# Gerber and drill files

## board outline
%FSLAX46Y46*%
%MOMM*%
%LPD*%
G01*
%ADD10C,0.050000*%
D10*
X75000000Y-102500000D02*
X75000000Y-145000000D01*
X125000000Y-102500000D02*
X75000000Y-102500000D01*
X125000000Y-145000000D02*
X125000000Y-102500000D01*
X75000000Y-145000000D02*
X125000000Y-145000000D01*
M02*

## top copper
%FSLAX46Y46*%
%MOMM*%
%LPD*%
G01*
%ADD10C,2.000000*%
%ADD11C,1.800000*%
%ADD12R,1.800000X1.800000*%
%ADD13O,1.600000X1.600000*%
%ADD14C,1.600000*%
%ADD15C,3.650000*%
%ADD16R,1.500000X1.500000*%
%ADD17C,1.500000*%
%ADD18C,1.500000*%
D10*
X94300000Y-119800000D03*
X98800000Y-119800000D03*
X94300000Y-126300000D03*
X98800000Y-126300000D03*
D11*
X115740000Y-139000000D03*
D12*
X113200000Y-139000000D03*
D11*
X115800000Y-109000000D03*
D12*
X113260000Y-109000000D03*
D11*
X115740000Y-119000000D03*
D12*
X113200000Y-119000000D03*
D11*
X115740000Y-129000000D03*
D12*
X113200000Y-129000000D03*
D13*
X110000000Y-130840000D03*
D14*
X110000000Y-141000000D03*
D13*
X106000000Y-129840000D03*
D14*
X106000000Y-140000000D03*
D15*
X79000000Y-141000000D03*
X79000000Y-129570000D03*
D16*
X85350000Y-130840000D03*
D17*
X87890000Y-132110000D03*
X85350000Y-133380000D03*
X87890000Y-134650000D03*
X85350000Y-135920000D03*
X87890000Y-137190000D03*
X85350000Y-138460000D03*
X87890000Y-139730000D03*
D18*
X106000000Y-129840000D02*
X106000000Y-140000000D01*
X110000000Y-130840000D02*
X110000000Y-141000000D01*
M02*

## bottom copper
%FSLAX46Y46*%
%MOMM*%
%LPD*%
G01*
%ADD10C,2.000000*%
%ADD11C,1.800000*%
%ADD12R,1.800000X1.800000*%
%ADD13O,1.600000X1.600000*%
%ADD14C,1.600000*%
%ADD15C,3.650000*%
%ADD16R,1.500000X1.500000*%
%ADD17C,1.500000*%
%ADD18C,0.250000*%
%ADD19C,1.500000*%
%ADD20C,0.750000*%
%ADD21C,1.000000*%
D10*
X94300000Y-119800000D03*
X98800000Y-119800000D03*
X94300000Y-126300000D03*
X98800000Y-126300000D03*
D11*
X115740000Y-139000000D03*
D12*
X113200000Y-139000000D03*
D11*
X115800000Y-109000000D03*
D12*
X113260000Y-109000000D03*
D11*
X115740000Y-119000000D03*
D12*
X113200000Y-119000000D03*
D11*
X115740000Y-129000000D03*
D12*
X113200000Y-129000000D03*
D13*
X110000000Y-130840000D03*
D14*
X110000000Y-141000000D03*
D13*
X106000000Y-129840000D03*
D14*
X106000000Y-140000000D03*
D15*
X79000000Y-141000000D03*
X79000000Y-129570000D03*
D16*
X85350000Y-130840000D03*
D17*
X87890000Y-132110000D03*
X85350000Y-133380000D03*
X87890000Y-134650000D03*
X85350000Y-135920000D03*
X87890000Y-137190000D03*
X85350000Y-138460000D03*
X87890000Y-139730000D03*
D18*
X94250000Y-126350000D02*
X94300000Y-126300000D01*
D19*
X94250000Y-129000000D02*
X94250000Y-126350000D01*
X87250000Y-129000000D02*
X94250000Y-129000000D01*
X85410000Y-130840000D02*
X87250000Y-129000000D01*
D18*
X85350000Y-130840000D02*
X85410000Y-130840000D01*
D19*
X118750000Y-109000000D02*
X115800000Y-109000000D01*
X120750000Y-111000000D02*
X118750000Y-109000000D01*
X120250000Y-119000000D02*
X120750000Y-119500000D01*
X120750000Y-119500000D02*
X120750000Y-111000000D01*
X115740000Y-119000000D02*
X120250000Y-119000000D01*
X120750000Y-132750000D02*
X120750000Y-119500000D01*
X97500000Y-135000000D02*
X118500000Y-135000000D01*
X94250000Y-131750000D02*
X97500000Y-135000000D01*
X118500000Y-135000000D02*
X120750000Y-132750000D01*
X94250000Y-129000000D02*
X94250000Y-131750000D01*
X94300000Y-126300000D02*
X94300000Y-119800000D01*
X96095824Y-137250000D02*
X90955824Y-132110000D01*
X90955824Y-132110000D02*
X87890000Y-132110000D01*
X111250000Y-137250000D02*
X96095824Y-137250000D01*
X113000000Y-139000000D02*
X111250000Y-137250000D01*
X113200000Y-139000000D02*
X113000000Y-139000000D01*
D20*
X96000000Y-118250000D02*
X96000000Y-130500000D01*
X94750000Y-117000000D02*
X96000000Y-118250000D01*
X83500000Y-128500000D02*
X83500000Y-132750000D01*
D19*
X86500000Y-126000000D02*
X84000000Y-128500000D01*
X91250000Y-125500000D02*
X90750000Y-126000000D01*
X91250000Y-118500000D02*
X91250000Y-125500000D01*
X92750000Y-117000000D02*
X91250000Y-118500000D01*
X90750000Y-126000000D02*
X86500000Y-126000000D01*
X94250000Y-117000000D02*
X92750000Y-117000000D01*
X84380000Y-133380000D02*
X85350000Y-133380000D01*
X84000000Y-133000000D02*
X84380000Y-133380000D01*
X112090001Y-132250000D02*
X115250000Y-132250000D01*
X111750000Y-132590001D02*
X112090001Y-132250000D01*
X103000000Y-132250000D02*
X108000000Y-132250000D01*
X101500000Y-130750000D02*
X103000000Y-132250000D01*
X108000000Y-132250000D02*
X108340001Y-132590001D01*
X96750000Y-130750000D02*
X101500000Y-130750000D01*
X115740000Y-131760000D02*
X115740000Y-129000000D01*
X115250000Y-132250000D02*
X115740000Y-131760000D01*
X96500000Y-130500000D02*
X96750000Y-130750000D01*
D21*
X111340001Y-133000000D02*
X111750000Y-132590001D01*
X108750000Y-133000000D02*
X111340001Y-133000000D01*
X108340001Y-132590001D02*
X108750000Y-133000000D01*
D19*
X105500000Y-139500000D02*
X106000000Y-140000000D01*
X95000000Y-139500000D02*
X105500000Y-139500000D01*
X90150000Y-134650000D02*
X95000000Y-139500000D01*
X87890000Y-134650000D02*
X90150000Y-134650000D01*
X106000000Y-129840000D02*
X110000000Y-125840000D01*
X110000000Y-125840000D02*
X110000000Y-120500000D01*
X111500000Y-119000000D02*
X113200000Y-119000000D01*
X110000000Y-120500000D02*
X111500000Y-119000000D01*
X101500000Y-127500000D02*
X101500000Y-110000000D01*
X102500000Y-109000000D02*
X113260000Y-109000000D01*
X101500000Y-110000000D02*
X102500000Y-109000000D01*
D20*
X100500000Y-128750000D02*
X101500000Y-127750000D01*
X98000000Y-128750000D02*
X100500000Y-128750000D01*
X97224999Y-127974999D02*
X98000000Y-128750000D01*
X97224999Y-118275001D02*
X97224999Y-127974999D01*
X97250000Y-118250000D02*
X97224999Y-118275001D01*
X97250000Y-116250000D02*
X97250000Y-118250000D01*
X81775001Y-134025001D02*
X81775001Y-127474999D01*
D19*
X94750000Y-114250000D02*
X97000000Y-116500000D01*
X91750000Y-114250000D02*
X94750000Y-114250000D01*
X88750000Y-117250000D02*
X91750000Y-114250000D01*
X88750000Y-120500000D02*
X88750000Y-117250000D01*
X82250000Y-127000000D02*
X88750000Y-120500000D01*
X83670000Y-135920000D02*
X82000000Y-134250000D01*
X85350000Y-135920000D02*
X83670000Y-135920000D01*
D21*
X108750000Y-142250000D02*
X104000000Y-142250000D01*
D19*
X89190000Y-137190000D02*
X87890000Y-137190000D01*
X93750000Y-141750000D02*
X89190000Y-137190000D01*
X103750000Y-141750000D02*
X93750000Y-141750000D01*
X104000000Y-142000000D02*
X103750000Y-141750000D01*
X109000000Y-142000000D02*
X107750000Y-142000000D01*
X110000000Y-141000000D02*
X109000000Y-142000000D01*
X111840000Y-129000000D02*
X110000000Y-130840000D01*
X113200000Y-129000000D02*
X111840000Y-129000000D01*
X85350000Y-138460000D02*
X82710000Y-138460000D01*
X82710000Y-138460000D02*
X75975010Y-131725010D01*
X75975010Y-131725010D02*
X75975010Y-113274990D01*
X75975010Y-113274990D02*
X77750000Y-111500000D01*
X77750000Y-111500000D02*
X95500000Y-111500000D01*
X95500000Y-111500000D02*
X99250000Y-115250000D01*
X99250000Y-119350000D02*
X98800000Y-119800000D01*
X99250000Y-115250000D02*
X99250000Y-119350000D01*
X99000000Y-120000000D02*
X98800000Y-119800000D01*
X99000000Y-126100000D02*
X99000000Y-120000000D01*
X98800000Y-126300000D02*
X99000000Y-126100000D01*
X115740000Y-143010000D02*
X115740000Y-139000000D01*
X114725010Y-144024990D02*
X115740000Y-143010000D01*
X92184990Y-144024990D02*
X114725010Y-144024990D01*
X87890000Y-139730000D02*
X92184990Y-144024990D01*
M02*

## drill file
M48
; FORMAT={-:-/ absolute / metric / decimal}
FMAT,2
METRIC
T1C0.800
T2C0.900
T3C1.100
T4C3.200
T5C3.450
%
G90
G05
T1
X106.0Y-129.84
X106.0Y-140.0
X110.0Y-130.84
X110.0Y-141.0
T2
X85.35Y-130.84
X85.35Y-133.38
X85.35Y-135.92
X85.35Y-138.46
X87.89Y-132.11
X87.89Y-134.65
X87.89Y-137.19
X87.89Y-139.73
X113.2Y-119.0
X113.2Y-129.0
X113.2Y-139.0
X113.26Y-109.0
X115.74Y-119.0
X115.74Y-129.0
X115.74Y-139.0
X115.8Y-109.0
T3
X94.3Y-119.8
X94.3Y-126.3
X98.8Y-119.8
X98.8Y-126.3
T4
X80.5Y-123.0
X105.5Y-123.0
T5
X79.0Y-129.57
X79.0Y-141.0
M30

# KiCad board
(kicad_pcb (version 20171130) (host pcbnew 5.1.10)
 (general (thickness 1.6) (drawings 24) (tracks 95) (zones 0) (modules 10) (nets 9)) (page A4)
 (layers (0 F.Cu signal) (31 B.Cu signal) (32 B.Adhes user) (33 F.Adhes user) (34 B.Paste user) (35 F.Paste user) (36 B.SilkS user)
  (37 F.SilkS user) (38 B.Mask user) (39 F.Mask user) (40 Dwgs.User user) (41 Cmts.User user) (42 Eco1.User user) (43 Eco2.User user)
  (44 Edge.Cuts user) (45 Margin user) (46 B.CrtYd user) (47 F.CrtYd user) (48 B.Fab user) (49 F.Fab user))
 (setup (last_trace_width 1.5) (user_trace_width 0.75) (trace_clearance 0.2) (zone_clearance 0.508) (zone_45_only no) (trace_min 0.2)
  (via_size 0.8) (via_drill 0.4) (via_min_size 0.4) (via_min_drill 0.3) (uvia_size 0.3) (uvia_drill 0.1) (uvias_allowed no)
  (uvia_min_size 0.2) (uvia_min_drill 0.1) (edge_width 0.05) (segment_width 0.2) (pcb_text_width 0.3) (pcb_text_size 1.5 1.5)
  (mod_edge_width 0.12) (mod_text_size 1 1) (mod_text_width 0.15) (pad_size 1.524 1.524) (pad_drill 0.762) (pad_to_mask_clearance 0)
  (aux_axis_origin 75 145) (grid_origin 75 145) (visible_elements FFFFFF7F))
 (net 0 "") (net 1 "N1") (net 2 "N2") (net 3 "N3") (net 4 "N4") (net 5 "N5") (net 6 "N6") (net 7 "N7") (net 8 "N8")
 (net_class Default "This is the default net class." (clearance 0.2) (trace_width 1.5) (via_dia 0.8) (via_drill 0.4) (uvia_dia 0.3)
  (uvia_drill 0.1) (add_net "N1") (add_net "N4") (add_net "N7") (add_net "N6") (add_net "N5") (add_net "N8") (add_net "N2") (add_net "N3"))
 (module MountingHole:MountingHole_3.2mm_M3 (layer F.Cu) (at 105.5 123)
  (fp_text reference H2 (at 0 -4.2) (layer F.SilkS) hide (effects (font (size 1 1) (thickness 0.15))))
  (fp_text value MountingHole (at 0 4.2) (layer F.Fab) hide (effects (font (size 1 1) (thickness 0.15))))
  (pad 1 np_thru_hole circle (at 0 0) (size 3.2 3.2) (drill 3.2) (layers *.Cu *.Mask)))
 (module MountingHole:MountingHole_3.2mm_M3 (layer F.Cu) (at 80.5 123)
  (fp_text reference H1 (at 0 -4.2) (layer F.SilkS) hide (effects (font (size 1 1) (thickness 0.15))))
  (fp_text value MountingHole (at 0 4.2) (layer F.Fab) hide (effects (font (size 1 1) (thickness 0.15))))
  (pad 1 np_thru_hole circle (at 0 0) (size 3.2 3.2) (drill 3.2) (layers *.Cu *.Mask)))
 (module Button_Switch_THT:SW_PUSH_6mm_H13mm (layer F.Cu) (at 94.3 126.3 90)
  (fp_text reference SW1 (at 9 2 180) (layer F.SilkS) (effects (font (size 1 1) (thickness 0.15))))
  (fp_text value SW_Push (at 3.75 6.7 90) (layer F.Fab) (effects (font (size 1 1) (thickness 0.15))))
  (pad 1 thru_hole circle (at 6.5 0 180) (size 2 2) (drill 1.1) (layers *.Cu *.Mask) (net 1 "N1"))
  (pad 2 thru_hole circle (at 6.5 4.5 180) (size 2 2) (drill 1.1) (layers *.Cu *.Mask) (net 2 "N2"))
  (pad 1 thru_hole circle (at 0 0 180) (size 2 2) (drill 1.1) (layers *.Cu *.Mask) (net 1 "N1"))
  (pad 2 thru_hole circle (at 0 4.5 180) (size 2 2) (drill 1.1) (layers *.Cu *.Mask) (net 2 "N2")))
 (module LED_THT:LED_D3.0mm (layer F.Cu) (at 113.2 139)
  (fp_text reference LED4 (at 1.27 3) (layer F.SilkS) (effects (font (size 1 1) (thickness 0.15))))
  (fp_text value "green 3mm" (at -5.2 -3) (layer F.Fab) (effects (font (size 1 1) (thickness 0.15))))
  (pad 2 thru_hole circle (at 2.54 0) (size 1.8 1.8) (drill 0.9) (layers *.Cu *.Mask) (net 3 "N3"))
  (pad 1 thru_hole rect (at 0 0) (size 1.8 1.8) (drill 0.9) (layers *.Cu *.Mask) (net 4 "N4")))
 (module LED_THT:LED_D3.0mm (layer F.Cu) (at 113.26 109)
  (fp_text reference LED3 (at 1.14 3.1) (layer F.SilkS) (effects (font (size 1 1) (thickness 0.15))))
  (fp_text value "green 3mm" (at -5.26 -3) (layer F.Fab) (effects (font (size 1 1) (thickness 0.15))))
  (pad 2 thru_hole circle (at 2.54 0) (size 1.8 1.8) (drill 0.9) (layers *.Cu *.Mask) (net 1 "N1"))
  (pad 1 thru_hole rect (at 0 0) (size 1.8 1.8) (drill 0.9) (layers *.Cu *.Mask) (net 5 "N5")))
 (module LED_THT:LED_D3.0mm (layer F.Cu) (at 113.2 119)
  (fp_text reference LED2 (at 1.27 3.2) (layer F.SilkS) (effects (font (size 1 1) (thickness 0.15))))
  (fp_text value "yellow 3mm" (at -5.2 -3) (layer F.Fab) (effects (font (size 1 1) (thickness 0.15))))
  (pad 2 thru_hole circle (at 2.54 0) (size 1.8 1.8) (drill 0.9) (layers *.Cu *.Mask) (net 1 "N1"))
  (pad 1 thru_hole rect (at 0 0) (size 1.8 1.8) (drill 0.9) (layers *.Cu *.Mask) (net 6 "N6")))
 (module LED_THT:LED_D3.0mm (layer F.Cu) (at 113.2 129)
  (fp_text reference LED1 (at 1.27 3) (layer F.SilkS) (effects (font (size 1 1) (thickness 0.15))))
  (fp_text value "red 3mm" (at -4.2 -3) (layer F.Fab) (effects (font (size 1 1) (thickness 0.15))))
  (pad 2 thru_hole circle (at 2.54 0) (size 1.8 1.8) (drill 0.9) (layers *.Cu *.Mask) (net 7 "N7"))
  (pad 1 thru_hole rect (at 0 0) (size 1.8 1.8) (drill 0.9) (layers *.Cu *.Mask) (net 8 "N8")))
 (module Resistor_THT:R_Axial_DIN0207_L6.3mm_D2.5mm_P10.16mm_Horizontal (layer F.Cu) (at 110 141 90)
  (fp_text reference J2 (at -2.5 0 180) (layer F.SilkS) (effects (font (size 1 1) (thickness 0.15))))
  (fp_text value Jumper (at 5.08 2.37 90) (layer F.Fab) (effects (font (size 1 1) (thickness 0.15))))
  (pad 2 thru_hole oval (at 10.16 0 90) (size 1.6 1.6) (drill 0.8) (layers *.Cu *.Mask) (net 8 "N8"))
  (pad 1 thru_hole circle (at 0 0 90) (size 1.6 1.6) (drill 0.8) (layers *.Cu *.Mask) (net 8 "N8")))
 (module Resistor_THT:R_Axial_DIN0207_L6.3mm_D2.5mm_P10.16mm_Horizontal (layer F.Cu) (at 106 140 90)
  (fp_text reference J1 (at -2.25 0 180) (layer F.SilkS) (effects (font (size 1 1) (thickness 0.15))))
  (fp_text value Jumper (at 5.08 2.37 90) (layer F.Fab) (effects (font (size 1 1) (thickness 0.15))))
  (pad 2 thru_hole oval (at 10.16 0 90) (size 1.6 1.6) (drill 0.8) (layers *.Cu *.Mask) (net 6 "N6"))
  (pad 1 thru_hole circle (at 0 0 90) (size 1.6 1.6) (drill 0.8) (layers *.Cu *.Mask) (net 6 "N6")))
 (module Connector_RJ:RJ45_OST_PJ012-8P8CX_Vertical (layer F.Cu) (at 85.35 130.84 270)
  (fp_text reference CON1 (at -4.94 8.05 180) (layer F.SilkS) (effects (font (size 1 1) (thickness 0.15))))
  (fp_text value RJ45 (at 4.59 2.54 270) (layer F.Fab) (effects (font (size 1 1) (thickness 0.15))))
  (pad "" np_thru_hole circle (at 10.16 6.35 270) (size 3.65 3.65) (drill 3.45) (layers *.Cu *.SilkS *.Mask))
  (pad "" np_thru_hole circle (at -1.27 6.35 270) (size 3.65 3.65) (drill 3.45) (layers *.Cu *.SilkS *.Mask))
  (pad 1 thru_hole rect (at 0 0 270) (size 1.5 1.5) (drill 0.9) (layers *.Cu *.Mask) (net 1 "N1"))
  (pad 2 thru_hole circle (at 1.27 -2.54 270) (size 1.5 1.5) (drill 0.9) (layers *.Cu *.Mask) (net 4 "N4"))
  (pad 3 thru_hole circle (at 2.54 0 270) (size 1.5 1.5) (drill 0.9) (layers *.Cu *.Mask) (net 7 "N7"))
  (pad 4 thru_hole circle (at 3.81 -2.54 270) (size 1.5 1.5) (drill 0.9) (layers *.Cu *.Mask) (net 6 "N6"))
  (pad 5 thru_hole circle (at 5.08 0 270) (size 1.5 1.5) (drill 0.9) (layers *.Cu *.Mask) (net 5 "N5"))
  (pad 6 thru_hole circle (at 6.35 -2.54 270) (size 1.5 1.5) (drill 0.9) (layers *.Cu *.Mask) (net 8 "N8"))
  (pad 7 thru_hole circle (at 7.62 0 270) (size 1.5 1.5) (drill 0.9) (layers *.Cu *.Mask) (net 2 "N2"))
  (pad 8 thru_hole circle (at 8.89 -2.54 270) (size 1.5 1.5) (drill 0.9) (layers *.Cu *.Mask) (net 3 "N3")))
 (gr_line (start 75 102.5) (end 75 145) (layer Edge.Cuts) (width 0.05))
 (gr_line (start 125 102.5) (end 75 102.5) (layer Edge.Cuts) (width 0.05))
 (gr_line (start 125 145) (end 125 102.5) (layer Edge.Cuts) (width 0.05))
 (gr_line (start 75 145) (end 125 145) (layer Edge.Cuts) (width 0.05))
 (segment (start 94.25 126.35) (end 94.3 126.3) (width 0.25) (layer B.Cu) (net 1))
 (segment (start 94.25 129) (end 94.25 126.35) (width 1.5) (layer B.Cu) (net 1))
 (segment (start 87.25 129) (end 94.25 129) (width 1.5) (layer B.Cu) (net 1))
 (segment (start 85.41 130.84) (end 87.25 129) (width 1.5) (layer B.Cu) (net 1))
 (segment (start 85.35 130.84) (end 85.41 130.84) (width 0.25) (layer B.Cu) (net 1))
 (segment (start 118.75 109) (end 115.8 109) (width 1.5) (layer B.Cu) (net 1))
 (segment (start 120.75 111) (end 118.75 109) (width 1.5) (layer B.Cu) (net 1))
 (segment (start 120.25 119) (end 120.75 119.5) (width 1.5) (layer B.Cu) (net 1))
 (segment (start 120.75 119.5) (end 120.75 111) (width 1.5) (layer B.Cu) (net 1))
 (segment (start 115.74 119) (end 120.25 119) (width 1.5) (layer B.Cu) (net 1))
 (segment (start 120.75 132.75) (end 120.75 119.5) (width 1.5) (layer B.Cu) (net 1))
 (segment (start 97.5 135) (end 118.5 135) (width 1.5) (layer B.Cu) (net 1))
 (segment (start 94.25 131.75) (end 97.5 135) (width 1.5) (layer B.Cu) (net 1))
 (segment (start 118.5 135) (end 120.75 132.75) (width 1.5) (layer B.Cu) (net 1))
 (segment (start 94.25 129) (end 94.25 131.75) (width 1.5) (layer B.Cu) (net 1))
 (segment (start 94.3 126.3) (end 94.3 119.8) (width 1.5) (layer B.Cu) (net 1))
 (segment (start 96.095824 137.25) (end 90.955824 132.11) (width 1.5) (layer B.Cu) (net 4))
 (segment (start 90.955824 132.11) (end 87.89 132.11) (width 1.5) (layer B.Cu) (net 4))
 (segment (start 111.25 137.25) (end 96.095824 137.25) (width 1.5) (layer B.Cu) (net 4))
 (segment (start 113 139) (end 111.25 137.25) (width 1.5) (layer B.Cu) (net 4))
 (segment (start 113.2 139) (end 113 139) (width 1.5) (layer B.Cu) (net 4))
 (segment (start 96 118.25) (end 96 130.5) (width 0.75) (layer B.Cu) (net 7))
 (segment (start 94.75 117) (end 96 118.25) (width 0.75) (layer B.Cu) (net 7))
 (segment (start 83.5 128.5) (end 83.5 132.75) (width 0.75) (layer B.Cu) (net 7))
 (segment (start 86.5 126) (end 84 128.5) (width 1.5) (layer B.Cu) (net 7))
 (segment (start 91.25 125.5) (end 90.75 126) (width 1.5) (layer B.Cu) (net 7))
 (segment (start 91.25 118.5) (end 91.25 125.5) (width 1.5) (layer B.Cu) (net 7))
 (segment (start 92.75 117) (end 91.25 118.5) (width 1.5) (layer B.Cu) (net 7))
 (segment (start 90.75 126) (end 86.5 126) (width 1.5) (layer B.Cu) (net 7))
 (segment (start 94.25 117) (end 92.75 117) (width 1.5) (layer B.Cu) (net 7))
 (segment (start 84.38 133.38) (end 85.35 133.38) (width 1.5) (layer B.Cu) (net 7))
 (segment (start 84 133) (end 84.38 133.38) (width 1.5) (layer B.Cu) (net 7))
 (segment (start 112.090001 132.25) (end 115.25 132.25) (width 1.5) (layer B.Cu) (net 7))
 (segment (start 111.75 132.590001) (end 112.090001 132.25) (width 1.5) (layer B.Cu) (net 7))
 (segment (start 103 132.25) (end 108 132.25) (width 1.5) (layer B.Cu) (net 7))
 (segment (start 101.5 130.75) (end 103 132.25) (width 1.5) (layer B.Cu) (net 7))
 (segment (start 108 132.25) (end 108.340001 132.590001) (width 1.5) (layer B.Cu) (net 7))
 (segment (start 96.75 130.75) (end 101.5 130.75) (width 1.5) (layer B.Cu) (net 7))
 (segment (start 115.74 131.76) (end 115.74 129) (width 1.5) (layer B.Cu) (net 7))
 (segment (start 115.25 132.25) (end 115.74 131.76) (width 1.5) (layer B.Cu) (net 7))
 (segment (start 96.5 130.5) (end 96.75 130.75) (width 1.5) (layer B.Cu) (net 7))
 (segment (start 111.340001 133) (end 111.75 132.590001) (width 1) (layer B.Cu) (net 7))
 (segment (start 108.75 133) (end 111.340001 133) (width 1) (layer B.Cu) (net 7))
 (segment (start 108.340001 132.590001) (end 108.75 133) (width 1) (layer B.Cu) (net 7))
 (segment (start 105.5 139.5) (end 106 140) (width 1.5) (layer B.Cu) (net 6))
 (segment (start 95 139.5) (end 105.5 139.5) (width 1.5) (layer B.Cu) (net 6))
 (segment (start 90.15 134.65) (end 95 139.5) (width 1.5) (layer B.Cu) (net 6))
 (segment (start 87.89 134.65) (end 90.15 134.65) (width 1.5) (layer B.Cu) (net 6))
 (segment (start 106 129.84) (end 110 125.84) (width 1.5) (layer B.Cu) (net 6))
 (segment (start 110 125.84) (end 110 120.5) (width 1.5) (layer B.Cu) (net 6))
 (segment (start 111.5 119) (end 113.2 119) (width 1.5) (layer B.Cu) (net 6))
 (segment (start 110 120.5) (end 111.5 119) (width 1.5) (layer B.Cu) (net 6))
 (segment (start 106 129.84) (end 106 140) (width 1.5) (layer F.Cu) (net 6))
 (segment (start 101.5 127.5) (end 101.5 110) (width 1.5) (layer B.Cu) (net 5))
 (segment (start 102.5 109) (end 113.26 109) (width 1.5) (layer B.Cu) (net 5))
 (segment (start 101.5 110) (end 102.5 109) (width 1.5) (layer B.Cu) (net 5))
 (segment (start 100.5 128.75) (end 101.5 127.75) (width 0.75) (layer B.Cu) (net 5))
 (segment (start 98 128.75) (end 100.5 128.75) (width 0.75) (layer B.Cu) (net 5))
 (segment (start 97.224999 127.974999) (end 98 128.75) (width 0.75) (layer B.Cu) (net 5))
 (segment (start 97.224999 118.275001) (end 97.224999 127.974999) (width 0.75) (layer B.Cu) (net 5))
 (segment (start 97.25 118.25) (end 97.224999 118.275001) (width 0.75) (layer B.Cu) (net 5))
 (segment (start 97.25 116.25) (end 97.25 118.25) (width 0.75) (layer B.Cu) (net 5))
 (segment (start 81.775001 134.025001) (end 81.775001 127.474999) (width 0.75) (layer B.Cu) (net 5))
 (segment (start 94.75 114.25) (end 97 116.5) (width 1.5) (layer B.Cu) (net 5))
 (segment (start 91.75 114.25) (end 94.75 114.25) (width 1.5) (layer B.Cu) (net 5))
 (segment (start 88.75 117.25) (end 91.75 114.25) (width 1.5) (layer B.Cu) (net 5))
 (segment (start 88.75 120.5) (end 88.75 117.25) (width 1.5) (layer B.Cu) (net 5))
 (segment (start 82.25 127) (end 88.75 120.5) (width 1.5) (layer B.Cu) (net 5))
 (segment (start 83.67 135.92) (end 82 134.25) (width 1.5) (layer B.Cu) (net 5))
 (segment (start 85.35 135.92) (end 83.67 135.92) (width 1.5) (layer B.Cu) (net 5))
 (segment (start 108.75 142.25) (end 104 142.25) (width 1) (layer B.Cu) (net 8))
 (segment (start 89.19 137.19) (end 87.89 137.19) (width 1.5) (layer B.Cu) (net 8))
 (segment (start 93.75 141.75) (end 89.19 137.19) (width 1.5) (layer B.Cu) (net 8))
 (segment (start 103.75 141.75) (end 93.75 141.75) (width 1.5) (layer B.Cu) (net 8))
 (segment (start 104 142) (end 103.75 141.75) (width 1.5) (layer B.Cu) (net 8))
 (segment (start 109 142) (end 107.75 142) (width 1.5) (layer B.Cu) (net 8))
 (segment (start 110 141) (end 109 142) (width 1.5) (layer B.Cu) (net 8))
 (segment (start 111.84 129) (end 110 130.84) (width 1.5) (layer B.Cu) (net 8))
 (segment (start 113.2 129) (end 111.84 129) (width 1.5) (layer B.Cu) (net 8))
 (segment (start 110 130.84) (end 110 141) (width 1.5) (layer F.Cu) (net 8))
 (segment (start 85.35 138.46) (end 82.71 138.46) (width 1.5) (layer B.Cu) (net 2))
 (segment (start 82.71 138.46) (end 75.97501 131.72501) (width 1.5) (layer B.Cu) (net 2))
 (segment (start 75.97501 131.72501) (end 75.97501 113.27499) (width 1.5) (layer B.Cu) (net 2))
 (segment (start 75.97501 113.27499) (end 77.75 111.5) (width 1.5) (layer B.Cu) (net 2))
 (segment (start 77.75 111.5) (end 95.5 111.5) (width 1.5) (layer B.Cu) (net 2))
 (segment (start 95.5 111.5) (end 99.25 115.25) (width 1.5) (layer B.Cu) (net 2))
 (segment (start 99.25 119.35) (end 98.8 119.8) (width 1.5) (layer B.Cu) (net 2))
 (segment (start 99.25 115.25) (end 99.25 119.35) (width 1.5) (layer B.Cu) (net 2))
 (segment (start 99 120) (end 98.8 119.8) (width 1.5) (layer B.Cu) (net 2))
 (segment (start 99 126.1) (end 99 120) (width 1.5) (layer B.Cu) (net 2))
 (segment (start 98.8 126.3) (end 99 126.1) (width 1.5) (layer B.Cu) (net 2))
 (segment (start 115.74 143.01) (end 115.74 139) (width 1.5) (layer B.Cu) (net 3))
 (segment (start 114.72501 144.02499) (end 115.74 143.01) (width 1.5) (layer B.Cu) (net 3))
 (segment (start 92.18499 144.02499) (end 114.72501 144.02499) (width 1.5) (layer B.Cu) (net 3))
 (segment (start 87.89 139.73) (end 92.18499 144.02499) (width 1.5) (layer B.Cu) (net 3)))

